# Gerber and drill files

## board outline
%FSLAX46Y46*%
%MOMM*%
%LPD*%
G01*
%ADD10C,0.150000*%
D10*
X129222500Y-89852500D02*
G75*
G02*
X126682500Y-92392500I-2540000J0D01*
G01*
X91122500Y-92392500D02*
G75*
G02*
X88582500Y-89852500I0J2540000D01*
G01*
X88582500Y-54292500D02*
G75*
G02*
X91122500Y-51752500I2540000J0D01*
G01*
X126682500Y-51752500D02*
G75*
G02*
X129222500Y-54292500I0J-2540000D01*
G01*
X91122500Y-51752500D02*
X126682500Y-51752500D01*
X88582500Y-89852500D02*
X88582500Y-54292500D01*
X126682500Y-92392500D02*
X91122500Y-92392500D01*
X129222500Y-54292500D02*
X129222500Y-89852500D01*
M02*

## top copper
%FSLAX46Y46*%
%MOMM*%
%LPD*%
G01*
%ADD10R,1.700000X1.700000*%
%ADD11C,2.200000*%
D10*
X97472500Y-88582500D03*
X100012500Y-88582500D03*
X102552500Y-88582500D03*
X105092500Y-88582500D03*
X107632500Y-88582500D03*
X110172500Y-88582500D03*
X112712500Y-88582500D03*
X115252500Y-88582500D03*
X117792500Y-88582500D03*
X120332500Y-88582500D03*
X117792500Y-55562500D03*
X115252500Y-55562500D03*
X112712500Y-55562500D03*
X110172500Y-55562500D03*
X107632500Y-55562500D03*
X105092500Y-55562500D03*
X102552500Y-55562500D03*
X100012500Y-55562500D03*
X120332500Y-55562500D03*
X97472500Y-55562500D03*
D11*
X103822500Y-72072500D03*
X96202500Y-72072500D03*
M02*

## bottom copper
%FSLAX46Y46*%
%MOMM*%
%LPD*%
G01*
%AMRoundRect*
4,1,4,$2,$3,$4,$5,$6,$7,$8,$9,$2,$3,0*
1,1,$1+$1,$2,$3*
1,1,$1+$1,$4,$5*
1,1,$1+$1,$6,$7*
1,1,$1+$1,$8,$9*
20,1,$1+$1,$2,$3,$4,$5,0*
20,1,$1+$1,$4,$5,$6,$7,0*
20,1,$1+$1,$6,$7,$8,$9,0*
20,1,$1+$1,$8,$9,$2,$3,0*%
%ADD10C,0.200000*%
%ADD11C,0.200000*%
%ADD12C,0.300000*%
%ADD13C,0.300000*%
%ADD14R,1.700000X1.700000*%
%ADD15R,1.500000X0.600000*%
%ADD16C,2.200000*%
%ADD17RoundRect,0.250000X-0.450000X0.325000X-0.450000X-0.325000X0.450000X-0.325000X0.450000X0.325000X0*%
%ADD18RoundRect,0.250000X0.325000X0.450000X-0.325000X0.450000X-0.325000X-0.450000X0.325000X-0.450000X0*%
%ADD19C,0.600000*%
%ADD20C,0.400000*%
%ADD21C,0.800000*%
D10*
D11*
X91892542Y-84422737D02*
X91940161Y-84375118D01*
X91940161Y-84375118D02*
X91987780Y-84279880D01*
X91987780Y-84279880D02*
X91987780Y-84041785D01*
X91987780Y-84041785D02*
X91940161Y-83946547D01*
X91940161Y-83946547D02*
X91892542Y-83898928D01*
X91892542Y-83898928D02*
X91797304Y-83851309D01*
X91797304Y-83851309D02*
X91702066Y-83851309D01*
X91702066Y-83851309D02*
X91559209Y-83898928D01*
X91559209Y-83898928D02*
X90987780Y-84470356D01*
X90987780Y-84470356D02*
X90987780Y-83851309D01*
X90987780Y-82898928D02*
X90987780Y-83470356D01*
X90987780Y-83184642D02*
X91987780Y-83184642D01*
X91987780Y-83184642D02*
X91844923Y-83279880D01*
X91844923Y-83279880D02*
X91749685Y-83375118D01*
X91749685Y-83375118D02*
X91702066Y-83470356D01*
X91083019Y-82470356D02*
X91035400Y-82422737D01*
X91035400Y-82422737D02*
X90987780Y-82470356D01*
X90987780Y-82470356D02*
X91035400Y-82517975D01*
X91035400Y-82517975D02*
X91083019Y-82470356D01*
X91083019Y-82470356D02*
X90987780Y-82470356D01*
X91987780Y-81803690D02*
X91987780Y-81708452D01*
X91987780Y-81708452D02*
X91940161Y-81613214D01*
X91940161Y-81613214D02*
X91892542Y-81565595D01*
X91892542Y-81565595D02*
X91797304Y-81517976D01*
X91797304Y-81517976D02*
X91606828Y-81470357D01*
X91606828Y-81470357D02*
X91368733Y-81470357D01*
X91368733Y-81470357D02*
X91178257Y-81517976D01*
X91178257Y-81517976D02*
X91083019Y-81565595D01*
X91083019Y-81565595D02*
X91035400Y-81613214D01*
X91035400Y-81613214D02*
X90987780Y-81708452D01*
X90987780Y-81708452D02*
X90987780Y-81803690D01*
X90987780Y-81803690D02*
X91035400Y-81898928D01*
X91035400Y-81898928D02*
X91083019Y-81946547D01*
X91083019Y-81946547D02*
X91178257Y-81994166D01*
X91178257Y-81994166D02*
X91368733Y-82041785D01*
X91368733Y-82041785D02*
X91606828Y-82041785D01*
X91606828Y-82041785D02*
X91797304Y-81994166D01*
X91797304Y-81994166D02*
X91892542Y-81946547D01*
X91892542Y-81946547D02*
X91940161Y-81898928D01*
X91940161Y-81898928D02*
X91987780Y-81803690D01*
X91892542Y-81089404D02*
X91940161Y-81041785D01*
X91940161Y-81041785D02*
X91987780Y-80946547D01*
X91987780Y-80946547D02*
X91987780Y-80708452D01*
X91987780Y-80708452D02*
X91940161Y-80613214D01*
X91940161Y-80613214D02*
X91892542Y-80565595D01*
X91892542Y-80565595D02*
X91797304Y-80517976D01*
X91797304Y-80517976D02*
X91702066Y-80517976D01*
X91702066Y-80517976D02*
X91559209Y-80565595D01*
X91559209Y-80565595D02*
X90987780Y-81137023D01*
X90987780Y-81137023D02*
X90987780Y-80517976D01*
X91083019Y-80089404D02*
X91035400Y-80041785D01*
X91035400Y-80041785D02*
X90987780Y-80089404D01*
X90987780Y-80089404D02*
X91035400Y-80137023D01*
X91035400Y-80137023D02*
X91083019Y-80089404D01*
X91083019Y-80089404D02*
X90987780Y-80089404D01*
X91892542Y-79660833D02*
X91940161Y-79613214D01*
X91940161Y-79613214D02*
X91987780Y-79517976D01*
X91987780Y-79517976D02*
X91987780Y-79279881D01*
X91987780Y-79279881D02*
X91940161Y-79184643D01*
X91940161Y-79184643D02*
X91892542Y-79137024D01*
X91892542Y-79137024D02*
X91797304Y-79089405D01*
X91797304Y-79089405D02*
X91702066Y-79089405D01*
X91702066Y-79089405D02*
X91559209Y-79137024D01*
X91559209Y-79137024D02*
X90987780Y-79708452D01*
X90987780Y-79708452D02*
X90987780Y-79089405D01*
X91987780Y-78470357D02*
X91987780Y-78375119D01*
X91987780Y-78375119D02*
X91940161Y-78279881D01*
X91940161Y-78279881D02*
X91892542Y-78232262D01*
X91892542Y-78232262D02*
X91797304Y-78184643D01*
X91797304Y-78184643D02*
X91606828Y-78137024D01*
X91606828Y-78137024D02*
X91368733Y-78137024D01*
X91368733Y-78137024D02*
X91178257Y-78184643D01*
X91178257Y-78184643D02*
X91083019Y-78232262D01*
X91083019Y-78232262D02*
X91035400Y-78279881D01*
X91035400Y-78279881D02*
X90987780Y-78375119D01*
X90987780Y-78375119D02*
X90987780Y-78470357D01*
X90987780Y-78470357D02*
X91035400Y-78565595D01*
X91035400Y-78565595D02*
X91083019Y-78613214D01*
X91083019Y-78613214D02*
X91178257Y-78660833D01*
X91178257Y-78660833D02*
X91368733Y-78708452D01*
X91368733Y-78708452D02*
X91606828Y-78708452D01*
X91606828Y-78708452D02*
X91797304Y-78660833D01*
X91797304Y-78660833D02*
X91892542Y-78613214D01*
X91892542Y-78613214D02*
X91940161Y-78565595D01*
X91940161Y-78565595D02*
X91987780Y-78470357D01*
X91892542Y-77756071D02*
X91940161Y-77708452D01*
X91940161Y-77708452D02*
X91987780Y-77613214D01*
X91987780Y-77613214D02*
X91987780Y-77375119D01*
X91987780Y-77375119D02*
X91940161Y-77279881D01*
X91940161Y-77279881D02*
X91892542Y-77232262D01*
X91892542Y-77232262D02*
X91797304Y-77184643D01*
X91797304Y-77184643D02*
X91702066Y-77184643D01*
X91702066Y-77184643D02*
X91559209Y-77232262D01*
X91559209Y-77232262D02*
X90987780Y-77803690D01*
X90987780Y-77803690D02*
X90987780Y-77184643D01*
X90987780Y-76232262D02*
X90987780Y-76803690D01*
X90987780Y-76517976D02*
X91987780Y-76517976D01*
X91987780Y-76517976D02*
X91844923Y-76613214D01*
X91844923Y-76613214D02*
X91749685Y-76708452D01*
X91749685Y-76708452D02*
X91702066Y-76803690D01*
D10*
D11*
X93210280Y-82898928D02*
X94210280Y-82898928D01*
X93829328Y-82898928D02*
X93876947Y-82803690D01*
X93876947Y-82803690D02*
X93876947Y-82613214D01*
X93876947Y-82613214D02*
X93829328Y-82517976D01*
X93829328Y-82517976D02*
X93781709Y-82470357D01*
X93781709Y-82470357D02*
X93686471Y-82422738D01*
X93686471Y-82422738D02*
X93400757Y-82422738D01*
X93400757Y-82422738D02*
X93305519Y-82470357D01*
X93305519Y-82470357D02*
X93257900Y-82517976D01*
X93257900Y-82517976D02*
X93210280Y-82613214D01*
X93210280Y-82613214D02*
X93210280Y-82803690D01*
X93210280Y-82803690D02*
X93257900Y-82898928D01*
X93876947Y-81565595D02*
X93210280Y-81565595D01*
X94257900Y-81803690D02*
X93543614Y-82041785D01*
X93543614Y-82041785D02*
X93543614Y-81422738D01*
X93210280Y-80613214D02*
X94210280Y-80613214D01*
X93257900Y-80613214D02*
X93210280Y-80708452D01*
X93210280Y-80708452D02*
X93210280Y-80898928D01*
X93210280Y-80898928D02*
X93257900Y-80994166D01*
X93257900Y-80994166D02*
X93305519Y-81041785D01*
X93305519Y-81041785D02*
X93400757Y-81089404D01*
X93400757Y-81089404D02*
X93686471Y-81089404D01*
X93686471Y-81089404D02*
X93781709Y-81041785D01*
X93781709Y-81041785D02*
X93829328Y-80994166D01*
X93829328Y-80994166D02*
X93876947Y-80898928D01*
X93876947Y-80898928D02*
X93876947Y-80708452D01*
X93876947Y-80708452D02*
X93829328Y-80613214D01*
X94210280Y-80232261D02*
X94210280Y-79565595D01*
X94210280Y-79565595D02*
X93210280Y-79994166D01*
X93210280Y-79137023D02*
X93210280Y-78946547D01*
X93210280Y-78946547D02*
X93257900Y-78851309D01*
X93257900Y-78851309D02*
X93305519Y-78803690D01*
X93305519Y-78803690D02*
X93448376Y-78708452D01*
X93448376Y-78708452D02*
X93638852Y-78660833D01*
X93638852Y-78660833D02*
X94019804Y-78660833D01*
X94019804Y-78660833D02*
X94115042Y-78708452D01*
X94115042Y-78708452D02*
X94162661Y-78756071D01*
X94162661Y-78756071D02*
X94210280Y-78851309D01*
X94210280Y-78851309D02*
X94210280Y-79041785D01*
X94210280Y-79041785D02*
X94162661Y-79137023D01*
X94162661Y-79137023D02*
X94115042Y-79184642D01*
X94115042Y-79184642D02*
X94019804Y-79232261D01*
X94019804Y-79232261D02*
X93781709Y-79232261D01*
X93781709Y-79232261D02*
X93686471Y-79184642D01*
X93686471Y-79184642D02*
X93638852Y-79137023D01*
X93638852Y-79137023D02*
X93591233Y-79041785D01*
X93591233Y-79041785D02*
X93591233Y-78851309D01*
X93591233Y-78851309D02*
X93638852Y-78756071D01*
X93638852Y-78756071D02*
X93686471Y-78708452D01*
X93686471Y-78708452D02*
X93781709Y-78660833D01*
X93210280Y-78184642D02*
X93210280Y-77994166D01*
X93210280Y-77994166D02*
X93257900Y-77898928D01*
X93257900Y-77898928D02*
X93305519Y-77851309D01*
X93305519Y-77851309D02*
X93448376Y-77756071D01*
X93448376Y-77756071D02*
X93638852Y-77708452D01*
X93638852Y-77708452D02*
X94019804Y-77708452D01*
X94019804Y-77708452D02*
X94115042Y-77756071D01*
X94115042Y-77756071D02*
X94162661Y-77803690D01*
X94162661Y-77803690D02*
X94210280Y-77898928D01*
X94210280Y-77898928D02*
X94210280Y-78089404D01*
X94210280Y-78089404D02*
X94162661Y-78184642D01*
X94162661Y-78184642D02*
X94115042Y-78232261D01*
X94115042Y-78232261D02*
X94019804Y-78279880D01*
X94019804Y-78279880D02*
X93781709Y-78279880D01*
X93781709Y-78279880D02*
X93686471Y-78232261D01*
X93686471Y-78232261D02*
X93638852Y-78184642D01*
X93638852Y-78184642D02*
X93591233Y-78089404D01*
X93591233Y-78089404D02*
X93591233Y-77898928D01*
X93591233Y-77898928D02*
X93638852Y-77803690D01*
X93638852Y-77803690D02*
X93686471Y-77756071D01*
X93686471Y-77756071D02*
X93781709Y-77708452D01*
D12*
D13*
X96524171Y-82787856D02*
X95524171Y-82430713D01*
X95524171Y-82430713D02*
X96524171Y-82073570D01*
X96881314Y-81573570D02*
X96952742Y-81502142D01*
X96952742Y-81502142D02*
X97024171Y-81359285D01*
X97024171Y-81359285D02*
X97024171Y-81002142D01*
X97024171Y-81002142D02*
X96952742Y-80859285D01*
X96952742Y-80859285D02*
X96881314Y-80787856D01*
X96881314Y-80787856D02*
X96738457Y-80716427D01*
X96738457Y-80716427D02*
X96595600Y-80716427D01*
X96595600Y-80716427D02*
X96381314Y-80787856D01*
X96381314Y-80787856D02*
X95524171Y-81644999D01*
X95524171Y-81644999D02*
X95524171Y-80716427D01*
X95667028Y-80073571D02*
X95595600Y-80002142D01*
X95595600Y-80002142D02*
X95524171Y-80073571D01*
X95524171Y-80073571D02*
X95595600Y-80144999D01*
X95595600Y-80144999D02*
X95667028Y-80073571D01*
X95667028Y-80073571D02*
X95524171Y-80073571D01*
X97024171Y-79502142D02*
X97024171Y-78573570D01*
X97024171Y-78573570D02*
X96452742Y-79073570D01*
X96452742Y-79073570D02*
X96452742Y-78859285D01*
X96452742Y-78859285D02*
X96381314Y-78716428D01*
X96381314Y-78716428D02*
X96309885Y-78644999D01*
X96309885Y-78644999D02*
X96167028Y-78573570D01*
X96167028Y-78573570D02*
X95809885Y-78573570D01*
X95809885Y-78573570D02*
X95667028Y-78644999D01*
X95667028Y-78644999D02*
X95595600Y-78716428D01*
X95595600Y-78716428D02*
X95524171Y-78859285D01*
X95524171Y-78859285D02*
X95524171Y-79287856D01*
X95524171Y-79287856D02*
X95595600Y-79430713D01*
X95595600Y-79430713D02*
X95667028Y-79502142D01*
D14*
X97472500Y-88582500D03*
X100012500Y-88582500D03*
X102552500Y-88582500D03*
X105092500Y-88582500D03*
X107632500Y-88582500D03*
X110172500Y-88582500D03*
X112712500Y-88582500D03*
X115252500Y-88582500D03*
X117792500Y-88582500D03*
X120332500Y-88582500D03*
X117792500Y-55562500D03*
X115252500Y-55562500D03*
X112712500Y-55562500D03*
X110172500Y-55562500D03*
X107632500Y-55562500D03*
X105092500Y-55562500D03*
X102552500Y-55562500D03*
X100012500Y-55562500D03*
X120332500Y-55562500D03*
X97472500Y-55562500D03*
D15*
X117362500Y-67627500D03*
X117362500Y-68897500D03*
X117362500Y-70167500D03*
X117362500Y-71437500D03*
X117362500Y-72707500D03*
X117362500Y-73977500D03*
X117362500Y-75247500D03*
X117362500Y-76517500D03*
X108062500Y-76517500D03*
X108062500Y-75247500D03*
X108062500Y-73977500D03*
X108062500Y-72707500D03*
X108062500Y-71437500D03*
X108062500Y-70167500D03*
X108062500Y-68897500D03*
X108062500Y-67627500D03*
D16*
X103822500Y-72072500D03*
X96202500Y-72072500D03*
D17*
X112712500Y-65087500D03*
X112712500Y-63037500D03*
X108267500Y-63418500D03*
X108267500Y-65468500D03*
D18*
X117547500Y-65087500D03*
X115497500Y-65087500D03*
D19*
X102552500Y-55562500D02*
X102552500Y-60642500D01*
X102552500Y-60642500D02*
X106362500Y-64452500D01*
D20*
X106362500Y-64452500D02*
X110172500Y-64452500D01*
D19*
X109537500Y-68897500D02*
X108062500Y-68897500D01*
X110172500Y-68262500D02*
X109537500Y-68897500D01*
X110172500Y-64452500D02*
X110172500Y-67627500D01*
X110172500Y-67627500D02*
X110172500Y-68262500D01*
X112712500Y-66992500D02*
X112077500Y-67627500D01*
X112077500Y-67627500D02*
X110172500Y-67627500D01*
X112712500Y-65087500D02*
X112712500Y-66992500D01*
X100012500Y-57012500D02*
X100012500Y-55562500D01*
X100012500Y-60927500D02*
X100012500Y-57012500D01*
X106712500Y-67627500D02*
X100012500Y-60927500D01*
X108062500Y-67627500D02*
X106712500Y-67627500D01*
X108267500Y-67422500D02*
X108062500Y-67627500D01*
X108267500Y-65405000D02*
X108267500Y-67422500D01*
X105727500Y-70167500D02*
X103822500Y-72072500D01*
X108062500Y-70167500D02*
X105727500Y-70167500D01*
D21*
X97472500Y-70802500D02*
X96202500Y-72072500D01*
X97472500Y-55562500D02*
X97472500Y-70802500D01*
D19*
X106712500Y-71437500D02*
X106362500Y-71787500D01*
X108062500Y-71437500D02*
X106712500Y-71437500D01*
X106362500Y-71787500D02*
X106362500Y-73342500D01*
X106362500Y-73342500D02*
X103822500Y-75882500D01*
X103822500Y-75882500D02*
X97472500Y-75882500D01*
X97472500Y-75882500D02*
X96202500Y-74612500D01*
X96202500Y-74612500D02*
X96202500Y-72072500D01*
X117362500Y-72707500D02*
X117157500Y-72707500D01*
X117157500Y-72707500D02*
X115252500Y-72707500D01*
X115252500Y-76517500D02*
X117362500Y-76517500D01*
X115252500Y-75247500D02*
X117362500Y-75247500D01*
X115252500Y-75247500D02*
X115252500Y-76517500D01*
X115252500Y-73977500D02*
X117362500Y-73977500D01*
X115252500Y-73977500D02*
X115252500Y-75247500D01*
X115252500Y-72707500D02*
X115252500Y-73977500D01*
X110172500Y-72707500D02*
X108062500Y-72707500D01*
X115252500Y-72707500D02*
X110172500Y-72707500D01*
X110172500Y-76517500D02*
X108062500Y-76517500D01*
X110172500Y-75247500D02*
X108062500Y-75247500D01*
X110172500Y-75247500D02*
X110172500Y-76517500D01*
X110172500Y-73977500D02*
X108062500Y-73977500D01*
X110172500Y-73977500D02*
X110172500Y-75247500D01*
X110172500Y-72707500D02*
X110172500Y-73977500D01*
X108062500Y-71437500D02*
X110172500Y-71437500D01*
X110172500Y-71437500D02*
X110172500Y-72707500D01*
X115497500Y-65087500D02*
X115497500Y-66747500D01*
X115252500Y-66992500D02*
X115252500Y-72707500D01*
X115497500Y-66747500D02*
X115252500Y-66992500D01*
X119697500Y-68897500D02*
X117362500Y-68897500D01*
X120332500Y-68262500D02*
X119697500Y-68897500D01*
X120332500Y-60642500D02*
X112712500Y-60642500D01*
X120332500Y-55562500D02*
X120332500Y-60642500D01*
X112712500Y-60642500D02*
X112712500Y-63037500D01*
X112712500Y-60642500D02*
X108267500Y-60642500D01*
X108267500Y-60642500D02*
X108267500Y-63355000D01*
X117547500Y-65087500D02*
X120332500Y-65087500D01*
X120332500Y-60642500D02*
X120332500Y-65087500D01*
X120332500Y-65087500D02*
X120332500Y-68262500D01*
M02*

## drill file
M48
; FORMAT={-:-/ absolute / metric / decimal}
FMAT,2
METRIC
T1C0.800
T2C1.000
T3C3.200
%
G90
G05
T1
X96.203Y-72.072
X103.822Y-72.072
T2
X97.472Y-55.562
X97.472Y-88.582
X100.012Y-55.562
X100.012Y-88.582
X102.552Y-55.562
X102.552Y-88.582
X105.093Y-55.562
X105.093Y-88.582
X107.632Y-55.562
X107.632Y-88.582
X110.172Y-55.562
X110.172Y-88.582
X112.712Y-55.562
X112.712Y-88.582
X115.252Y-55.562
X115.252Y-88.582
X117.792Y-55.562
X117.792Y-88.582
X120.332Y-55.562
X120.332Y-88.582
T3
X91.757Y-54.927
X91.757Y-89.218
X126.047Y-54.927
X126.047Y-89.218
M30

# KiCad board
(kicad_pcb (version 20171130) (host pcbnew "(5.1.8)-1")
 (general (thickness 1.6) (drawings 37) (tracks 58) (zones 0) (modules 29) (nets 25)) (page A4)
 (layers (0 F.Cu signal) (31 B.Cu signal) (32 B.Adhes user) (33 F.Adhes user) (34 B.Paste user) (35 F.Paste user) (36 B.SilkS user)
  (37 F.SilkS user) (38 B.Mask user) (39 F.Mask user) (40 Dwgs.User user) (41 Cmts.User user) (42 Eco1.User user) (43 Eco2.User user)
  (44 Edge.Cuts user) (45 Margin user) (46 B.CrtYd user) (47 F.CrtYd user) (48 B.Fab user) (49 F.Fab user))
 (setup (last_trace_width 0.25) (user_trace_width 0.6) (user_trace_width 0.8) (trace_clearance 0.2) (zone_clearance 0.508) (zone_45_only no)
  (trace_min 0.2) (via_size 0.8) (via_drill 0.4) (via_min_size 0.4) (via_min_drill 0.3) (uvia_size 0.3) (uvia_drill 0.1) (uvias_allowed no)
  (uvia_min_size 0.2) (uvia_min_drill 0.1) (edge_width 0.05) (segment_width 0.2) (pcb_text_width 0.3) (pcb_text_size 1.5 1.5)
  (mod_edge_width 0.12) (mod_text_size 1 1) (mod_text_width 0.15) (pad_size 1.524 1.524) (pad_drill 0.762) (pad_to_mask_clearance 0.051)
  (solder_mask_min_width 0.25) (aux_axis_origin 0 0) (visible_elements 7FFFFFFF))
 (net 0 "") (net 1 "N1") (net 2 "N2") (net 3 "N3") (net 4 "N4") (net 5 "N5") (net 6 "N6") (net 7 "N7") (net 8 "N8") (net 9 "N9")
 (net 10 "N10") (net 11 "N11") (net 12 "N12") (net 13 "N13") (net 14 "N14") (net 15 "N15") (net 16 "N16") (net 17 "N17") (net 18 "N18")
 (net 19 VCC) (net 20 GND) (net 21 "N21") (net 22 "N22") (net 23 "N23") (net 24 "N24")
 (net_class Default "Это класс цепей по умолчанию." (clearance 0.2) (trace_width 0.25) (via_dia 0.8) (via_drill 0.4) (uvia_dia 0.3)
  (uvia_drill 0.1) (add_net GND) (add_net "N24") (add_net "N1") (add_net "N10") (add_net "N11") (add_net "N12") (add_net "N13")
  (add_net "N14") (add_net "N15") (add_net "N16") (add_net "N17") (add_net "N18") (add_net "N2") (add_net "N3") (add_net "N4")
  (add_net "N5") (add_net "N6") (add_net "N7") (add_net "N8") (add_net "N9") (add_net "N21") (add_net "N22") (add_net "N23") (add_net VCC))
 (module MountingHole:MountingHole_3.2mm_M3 (layer F.Cu) (at 126.0475 54.9275 270)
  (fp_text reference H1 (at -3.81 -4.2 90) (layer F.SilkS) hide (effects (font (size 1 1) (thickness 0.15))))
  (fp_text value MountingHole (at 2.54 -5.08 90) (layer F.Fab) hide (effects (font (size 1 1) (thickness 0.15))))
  (pad 1 np_thru_hole circle (at 0 0 270) (size 3.2 3.2) (drill 3.2) (layers *.Cu *.Mask)))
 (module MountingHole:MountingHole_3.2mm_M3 (layer F.Cu) (at 91.7575 54.9275 270)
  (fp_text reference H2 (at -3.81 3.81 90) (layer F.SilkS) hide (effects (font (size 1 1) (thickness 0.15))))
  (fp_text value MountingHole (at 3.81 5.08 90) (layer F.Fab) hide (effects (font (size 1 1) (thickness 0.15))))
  (pad 1 np_thru_hole circle (at 0 0 270) (size 3.2 3.2) (drill 3.2) (layers *.Cu *.Mask)))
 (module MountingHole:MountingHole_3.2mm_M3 (layer F.Cu) (at 126.0475 89.2175 270)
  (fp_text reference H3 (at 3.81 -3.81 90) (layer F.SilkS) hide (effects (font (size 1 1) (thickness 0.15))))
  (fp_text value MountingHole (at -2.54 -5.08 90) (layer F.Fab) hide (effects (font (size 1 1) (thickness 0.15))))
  (pad 1 np_thru_hole circle (at 0 0 270) (size 3.2 3.2) (drill 3.2) (layers *.Cu *.Mask)))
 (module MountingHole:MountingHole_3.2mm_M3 (layer F.Cu) (at 91.7575 89.2175 270)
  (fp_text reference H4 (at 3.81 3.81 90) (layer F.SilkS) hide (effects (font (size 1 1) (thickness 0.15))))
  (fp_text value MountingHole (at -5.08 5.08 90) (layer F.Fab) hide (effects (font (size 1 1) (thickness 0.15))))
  (pad 1 np_thru_hole circle (at 0 0 270) (size 3.2 3.2) (drill 3.2) (layers *.Cu *.Mask)))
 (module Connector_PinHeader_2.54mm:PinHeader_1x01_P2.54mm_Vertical (layer F.Cu) (at 97.4725 88.5825 270)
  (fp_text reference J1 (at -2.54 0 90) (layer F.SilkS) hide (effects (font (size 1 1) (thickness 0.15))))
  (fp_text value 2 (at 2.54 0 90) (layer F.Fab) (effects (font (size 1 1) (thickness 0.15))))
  (pad 1 thru_hole rect (at 0 0 270) (size 1.7 1.7) (drill 1) (layers *.Cu *.Mask) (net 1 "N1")))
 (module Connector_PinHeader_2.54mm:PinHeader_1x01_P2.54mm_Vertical (layer F.Cu) (at 100.0125 88.5825 270)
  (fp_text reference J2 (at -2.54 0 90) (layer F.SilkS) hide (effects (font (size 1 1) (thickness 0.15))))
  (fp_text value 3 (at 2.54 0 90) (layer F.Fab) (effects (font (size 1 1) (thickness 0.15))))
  (pad 1 thru_hole rect (at 0 0 270) (size 1.7 1.7) (drill 1) (layers *.Cu *.Mask) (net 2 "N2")))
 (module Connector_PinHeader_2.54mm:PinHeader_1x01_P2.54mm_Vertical (layer F.Cu) (at 102.5525 88.5825 270)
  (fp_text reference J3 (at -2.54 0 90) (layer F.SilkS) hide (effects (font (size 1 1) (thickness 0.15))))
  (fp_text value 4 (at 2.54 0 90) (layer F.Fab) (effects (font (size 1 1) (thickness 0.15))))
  (pad 1 thru_hole rect (at 0 0 270) (size 1.7 1.7) (drill 1) (layers *.Cu *.Mask) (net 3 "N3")))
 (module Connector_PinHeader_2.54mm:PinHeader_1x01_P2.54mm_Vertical (layer F.Cu) (at 105.0925 88.5825 270)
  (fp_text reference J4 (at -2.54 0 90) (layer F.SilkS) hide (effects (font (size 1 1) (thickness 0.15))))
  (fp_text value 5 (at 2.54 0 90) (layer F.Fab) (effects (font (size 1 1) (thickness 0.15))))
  (pad 1 thru_hole rect (at 0 0 270) (size 1.7 1.7) (drill 1) (layers *.Cu *.Mask) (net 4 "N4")))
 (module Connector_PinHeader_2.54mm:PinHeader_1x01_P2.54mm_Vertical (layer F.Cu) (at 107.6325 88.5825 270)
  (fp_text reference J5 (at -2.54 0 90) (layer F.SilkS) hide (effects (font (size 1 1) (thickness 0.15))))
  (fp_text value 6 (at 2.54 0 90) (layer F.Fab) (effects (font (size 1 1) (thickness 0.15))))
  (pad 1 thru_hole rect (at 0 0 270) (size 1.7 1.7) (drill 1) (layers *.Cu *.Mask) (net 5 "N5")))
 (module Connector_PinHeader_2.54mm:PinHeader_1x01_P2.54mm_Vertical (layer F.Cu) (at 110.1725 88.5825 270)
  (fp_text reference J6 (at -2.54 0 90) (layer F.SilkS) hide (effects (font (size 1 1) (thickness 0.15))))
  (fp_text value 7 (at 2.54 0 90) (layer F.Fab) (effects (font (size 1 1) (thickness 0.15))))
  (pad 1 thru_hole rect (at 0 0 270) (size 1.7 1.7) (drill 1) (layers *.Cu *.Mask) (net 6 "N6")))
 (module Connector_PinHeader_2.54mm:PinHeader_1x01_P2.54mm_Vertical (layer F.Cu) (at 112.7125 88.5825 270)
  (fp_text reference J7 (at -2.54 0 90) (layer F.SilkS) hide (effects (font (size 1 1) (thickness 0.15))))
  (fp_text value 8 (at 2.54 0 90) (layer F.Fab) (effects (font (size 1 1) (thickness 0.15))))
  (pad 1 thru_hole rect (at 0 0 270) (size 1.7 1.7) (drill 1) (layers *.Cu *.Mask) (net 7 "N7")))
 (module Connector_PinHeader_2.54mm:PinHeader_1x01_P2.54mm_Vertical (layer F.Cu) (at 115.2525 88.5825 270)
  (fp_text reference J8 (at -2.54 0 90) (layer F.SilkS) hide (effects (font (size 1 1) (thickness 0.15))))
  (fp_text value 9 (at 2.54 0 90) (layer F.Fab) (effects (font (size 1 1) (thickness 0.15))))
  (pad 1 thru_hole rect (at 0 0 270) (size 1.7 1.7) (drill 1) (layers *.Cu *.Mask) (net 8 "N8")))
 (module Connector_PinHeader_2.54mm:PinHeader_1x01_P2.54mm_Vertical (layer F.Cu) (at 117.7925 88.5825 270)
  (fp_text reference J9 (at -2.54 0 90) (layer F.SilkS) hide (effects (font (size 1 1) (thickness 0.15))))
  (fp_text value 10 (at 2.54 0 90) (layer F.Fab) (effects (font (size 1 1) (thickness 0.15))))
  (pad 1 thru_hole rect (at 0 0 270) (size 1.7 1.7) (drill 1) (layers *.Cu *.Mask) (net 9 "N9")))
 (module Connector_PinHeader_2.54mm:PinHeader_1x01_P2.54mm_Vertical (layer F.Cu) (at 120.3325 88.5825 270)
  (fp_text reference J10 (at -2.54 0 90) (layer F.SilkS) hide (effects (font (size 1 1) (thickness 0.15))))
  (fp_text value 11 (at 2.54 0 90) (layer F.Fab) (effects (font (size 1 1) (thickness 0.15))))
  (pad 1 thru_hole rect (at 0 0 270) (size 1.7 1.7) (drill 1) (layers *.Cu *.Mask) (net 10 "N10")))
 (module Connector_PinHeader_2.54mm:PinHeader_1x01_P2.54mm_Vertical (layer F.Cu) (at 117.7925 55.5625 270)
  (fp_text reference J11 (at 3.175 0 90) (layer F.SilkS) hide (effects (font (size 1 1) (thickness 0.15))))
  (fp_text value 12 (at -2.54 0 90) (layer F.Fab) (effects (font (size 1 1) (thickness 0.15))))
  (pad 1 thru_hole rect (at 0 0 270) (size 1.7 1.7) (drill 1) (layers *.Cu *.Mask) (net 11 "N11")))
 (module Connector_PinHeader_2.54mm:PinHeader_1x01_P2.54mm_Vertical (layer F.Cu) (at 115.2525 55.5625 270)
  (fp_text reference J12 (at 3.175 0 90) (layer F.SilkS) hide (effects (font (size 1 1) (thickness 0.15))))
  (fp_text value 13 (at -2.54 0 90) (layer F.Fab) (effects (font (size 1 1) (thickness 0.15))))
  (pad 1 thru_hole rect (at 0 0 270) (size 1.7 1.7) (drill 1) (layers *.Cu *.Mask) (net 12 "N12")))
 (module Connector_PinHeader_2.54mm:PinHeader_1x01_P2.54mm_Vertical (layer F.Cu) (at 112.7125 55.5625 270)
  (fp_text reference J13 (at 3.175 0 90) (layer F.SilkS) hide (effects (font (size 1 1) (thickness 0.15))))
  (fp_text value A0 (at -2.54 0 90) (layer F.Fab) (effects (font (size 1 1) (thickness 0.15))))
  (pad 1 thru_hole rect (at 0 0 270) (size 1.7 1.7) (drill 1) (layers *.Cu *.Mask) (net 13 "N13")))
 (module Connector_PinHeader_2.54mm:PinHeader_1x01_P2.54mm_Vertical (layer F.Cu) (at 110.1725 55.5625 270)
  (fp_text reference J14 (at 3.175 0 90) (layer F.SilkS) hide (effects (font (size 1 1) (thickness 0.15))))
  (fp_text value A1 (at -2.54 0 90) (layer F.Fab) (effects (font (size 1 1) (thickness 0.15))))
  (pad 1 thru_hole rect (at 0 0 270) (size 1.7 1.7) (drill 1) (layers *.Cu *.Mask) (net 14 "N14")))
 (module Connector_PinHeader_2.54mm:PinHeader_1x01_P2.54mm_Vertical (layer F.Cu) (at 107.6325 55.5625 270)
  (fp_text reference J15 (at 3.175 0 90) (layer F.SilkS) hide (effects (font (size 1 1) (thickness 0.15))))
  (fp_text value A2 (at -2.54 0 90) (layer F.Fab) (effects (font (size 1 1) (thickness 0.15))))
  (pad 1 thru_hole rect (at 0 0 270) (size 1.7 1.7) (drill 1) (layers *.Cu *.Mask) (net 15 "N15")))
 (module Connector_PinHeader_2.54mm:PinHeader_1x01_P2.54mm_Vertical (layer F.Cu) (at 105.0925 55.5625 270)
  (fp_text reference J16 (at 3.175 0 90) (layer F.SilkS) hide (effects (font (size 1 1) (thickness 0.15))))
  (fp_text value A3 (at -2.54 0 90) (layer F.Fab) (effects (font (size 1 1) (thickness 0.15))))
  (pad 1 thru_hole rect (at 0 0 270) (size 1.7 1.7) (drill 1) (layers *.Cu *.Mask) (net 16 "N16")))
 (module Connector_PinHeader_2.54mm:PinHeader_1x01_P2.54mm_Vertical (layer F.Cu) (at 102.5525 55.5625 270)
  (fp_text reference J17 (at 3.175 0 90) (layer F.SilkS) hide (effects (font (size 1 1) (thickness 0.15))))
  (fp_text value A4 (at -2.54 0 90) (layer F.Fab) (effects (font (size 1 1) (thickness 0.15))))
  (pad 1 thru_hole rect (at 0 0 270) (size 1.7 1.7) (drill 1) (layers *.Cu *.Mask) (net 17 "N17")))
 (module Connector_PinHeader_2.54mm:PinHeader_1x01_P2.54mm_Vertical (layer F.Cu) (at 100.0125 55.5625 270)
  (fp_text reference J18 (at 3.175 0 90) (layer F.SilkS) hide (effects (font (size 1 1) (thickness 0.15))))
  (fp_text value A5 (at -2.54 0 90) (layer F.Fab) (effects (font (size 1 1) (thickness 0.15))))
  (pad 1 thru_hole rect (at 0 0 270) (size 1.7 1.7) (drill 1) (layers *.Cu *.Mask) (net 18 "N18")))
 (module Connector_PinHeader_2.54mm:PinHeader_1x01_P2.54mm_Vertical (layer F.Cu) (at 120.3325 55.5625 270)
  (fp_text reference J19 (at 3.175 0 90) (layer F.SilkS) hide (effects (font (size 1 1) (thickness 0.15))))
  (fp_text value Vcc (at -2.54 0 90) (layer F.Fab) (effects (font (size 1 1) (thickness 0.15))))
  (pad 1 thru_hole rect (at 0 0 270) (size 1.7 1.7) (drill 1) (layers *.Cu *.Mask) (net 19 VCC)))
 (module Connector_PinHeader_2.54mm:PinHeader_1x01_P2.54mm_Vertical (layer F.Cu) (at 97.4725 55.5625 270)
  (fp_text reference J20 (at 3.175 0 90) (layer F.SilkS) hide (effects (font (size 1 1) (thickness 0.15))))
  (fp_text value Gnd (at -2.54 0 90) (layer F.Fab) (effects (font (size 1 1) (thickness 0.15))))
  (pad 1 thru_hole rect (at 0 0 270) (size 1.7 1.7) (drill 1) (layers *.Cu *.Mask) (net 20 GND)))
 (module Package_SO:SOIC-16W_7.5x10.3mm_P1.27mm (layer B.Cu) (at 112.7125 72.0725 180)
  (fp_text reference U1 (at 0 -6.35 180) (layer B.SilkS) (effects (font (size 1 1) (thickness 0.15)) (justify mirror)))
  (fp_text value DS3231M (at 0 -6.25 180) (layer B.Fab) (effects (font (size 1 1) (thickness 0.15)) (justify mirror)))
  (pad 1 smd rect (at -4.65 4.445 180) (size 1.5 0.6) (layers B.Cu B.Paste B.Mask) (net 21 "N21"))
  (pad 2 smd rect (at -4.65 3.175 180) (size 1.5 0.6) (layers B.Cu B.Paste B.Mask) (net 19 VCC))
  (pad 3 smd rect (at -4.65 1.905 180) (size 1.5 0.6) (layers B.Cu B.Paste B.Mask) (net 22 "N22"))
  (pad 4 smd rect (at -4.65 0.635 180) (size 1.5 0.6) (layers B.Cu B.Paste B.Mask) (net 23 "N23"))
  (pad 5 smd rect (at -4.65 -0.635 180) (size 1.5 0.6) (layers B.Cu B.Paste B.Mask) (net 20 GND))
  (pad 6 smd rect (at -4.65 -1.905 180) (size 1.5 0.6) (layers B.Cu B.Paste B.Mask) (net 20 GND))
  (pad 7 smd rect (at -4.65 -3.175 180) (size 1.5 0.6) (layers B.Cu B.Paste B.Mask) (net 20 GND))
  (pad 8 smd rect (at -4.65 -4.445 180) (size 1.5 0.6) (layers B.Cu B.Paste B.Mask) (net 20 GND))
  (pad 9 smd rect (at 4.65 -4.445 180) (size 1.5 0.6) (layers B.Cu B.Paste B.Mask) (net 20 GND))
  (pad 10 smd rect (at 4.65 -3.175 180) (size 1.5 0.6) (layers B.Cu B.Paste B.Mask) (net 20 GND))
  (pad 11 smd rect (at 4.65 -1.905 180) (size 1.5 0.6) (layers B.Cu B.Paste B.Mask) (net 20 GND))
  (pad 12 smd rect (at 4.65 -0.635 180) (size 1.5 0.6) (layers B.Cu B.Paste B.Mask) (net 20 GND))
  (pad 13 smd rect (at 4.65 0.635 180) (size 1.5 0.6) (layers B.Cu B.Paste B.Mask) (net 20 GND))
  (pad 14 smd rect (at 4.65 1.905 180) (size 1.5 0.6) (layers B.Cu B.Paste B.Mask) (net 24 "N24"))
  (pad 15 smd rect (at 4.65 3.175 180) (size 1.5 0.6) (layers B.Cu B.Paste B.Mask) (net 17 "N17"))
  (pad 16 smd rect (at 4.65 4.445 180) (size 1.5 0.6) (layers B.Cu B.Paste B.Mask) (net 18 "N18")))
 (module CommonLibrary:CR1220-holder (layer F.Cu) (at 96.2025 72.0725 180)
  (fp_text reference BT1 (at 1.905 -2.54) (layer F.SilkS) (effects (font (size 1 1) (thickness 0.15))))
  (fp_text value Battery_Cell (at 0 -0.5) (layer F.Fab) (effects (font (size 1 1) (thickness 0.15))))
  (pad 1 thru_hole circle (at -7.62 0 180) (size 2.2 2.2) (drill 0.8) (layers *.Cu *.Mask) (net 24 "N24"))
  (pad 2 thru_hole circle (at 0 0 180) (size 2.2 2.2) (drill 0.8) (layers *.Cu *.Mask) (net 20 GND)))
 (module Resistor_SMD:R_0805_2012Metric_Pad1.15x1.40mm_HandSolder (layer B.Cu) (at 112.7125 64.0625 270)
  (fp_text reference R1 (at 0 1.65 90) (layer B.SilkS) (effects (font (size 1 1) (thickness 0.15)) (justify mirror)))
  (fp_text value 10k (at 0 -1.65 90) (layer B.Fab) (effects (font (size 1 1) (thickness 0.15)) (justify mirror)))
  (pad 2 smd roundrect (at 1.025 0 270) (size 1.15 1.4) (layers B.Cu B.Paste B.Mask) (roundrect_rratio 0.217391) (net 17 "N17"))
  (pad 1 smd roundrect (at -1.025 0 270) (size 1.15 1.4) (layers B.Cu B.Paste B.Mask) (roundrect_rratio 0.217391) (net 19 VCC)))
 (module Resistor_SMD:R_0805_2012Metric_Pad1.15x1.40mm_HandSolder (layer B.Cu) (at 108.2675 64.4435 270)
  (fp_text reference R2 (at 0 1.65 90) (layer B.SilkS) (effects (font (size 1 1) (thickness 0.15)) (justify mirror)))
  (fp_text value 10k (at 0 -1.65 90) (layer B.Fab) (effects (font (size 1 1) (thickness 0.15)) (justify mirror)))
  (pad 1 smd roundrect (at -1.025 0 270) (size 1.15 1.4) (layers B.Cu B.Paste B.Mask) (roundrect_rratio 0.217391) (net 19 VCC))
  (pad 2 smd roundrect (at 1.025 0 270) (size 1.15 1.4) (layers B.Cu B.Paste B.Mask) (roundrect_rratio 0.217391) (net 18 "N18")))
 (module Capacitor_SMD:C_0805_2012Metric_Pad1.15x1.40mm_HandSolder (layer B.Cu) (at 116.5225 65.0875 180)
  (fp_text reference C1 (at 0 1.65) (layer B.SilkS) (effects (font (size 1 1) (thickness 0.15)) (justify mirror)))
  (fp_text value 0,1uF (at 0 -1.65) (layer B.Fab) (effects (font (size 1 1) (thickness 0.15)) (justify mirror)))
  (pad 1 smd roundrect (at -1.025 0 180) (size 1.15 1.4) (layers B.Cu B.Paste B.Mask) (roundrect_rratio 0.217391) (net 19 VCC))
  (pad 2 smd roundrect (at 1.025 0 180) (size 1.15 1.4) (layers B.Cu B.Paste B.Mask) (roundrect_rratio 0.217391) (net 20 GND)))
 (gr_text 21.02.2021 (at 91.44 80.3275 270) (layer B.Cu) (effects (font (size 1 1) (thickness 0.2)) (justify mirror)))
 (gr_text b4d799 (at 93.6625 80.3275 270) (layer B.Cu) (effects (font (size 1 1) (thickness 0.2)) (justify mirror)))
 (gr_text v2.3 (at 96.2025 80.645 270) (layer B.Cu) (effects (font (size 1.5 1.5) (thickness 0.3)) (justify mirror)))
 (gr_arc (start 126.6825 89.8525) (end 126.6825 92.3925) (angle -90) (layer Edge.Cuts) (width 0.15))
 (gr_arc (start 91.1225 89.8525) (end 88.5825 89.8525) (angle -90) (layer Edge.Cuts) (width 0.15))
 (gr_arc (start 91.1225 54.2925) (end 91.1225 51.7525) (angle -90) (layer Edge.Cuts) (width 0.15))
 (gr_arc (start 126.6825 54.2925) (end 129.2225 54.2925) (angle -90) (layer Edge.Cuts) (width 0.15))
 (gr_line (start 91.1225 51.7525) (end 126.6825 51.7525) (layer Edge.Cuts) (width 0.15))
 (gr_line (start 88.5825 89.8525) (end 88.5825 54.2925) (layer Edge.Cuts) (width 0.15))
 (gr_line (start 126.6825 92.3925) (end 91.1225 92.3925) (layer Edge.Cuts) (width 0.15))
 (gr_line (start 129.2225 54.2925) (end 129.2225 89.8525) (layer Edge.Cuts) (width 0.15))
 (segment (start 102.5525 55.5625) (end 102.5525 60.6425) (width 0.6) (layer B.Cu) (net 17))
 (segment (start 102.5525 60.6425) (end 106.3625 64.4525) (width 0.6) (layer B.Cu) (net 17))
 (segment (start 106.3625 64.4525) (end 110.1725 64.4525) (width 0.4) (layer B.Cu) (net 17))
 (segment (start 109.5375 68.8975) (end 108.0625 68.8975) (width 0.6) (layer B.Cu) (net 17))
 (segment (start 110.1725 68.2625) (end 109.5375 68.8975) (width 0.6) (layer B.Cu) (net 17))
 (segment (start 110.1725 64.4525) (end 110.1725 67.6275) (width 0.6) (layer B.Cu) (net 17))
 (segment (start 110.1725 67.6275) (end 110.1725 68.2625) (width 0.6) (layer B.Cu) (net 17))
 (segment (start 112.7125 66.9925) (end 112.0775 67.6275) (width 0.6) (layer B.Cu) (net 17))
 (segment (start 112.0775 67.6275) (end 110.1725 67.6275) (width 0.6) (layer B.Cu) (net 17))
 (segment (start 112.7125 65.0875) (end 112.7125 66.9925) (width 0.6) (layer B.Cu) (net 17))
 (segment (start 100.0125 57.0125) (end 100.0125 55.5625) (width 0.6) (layer B.Cu) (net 18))
 (segment (start 100.0125 60.9275) (end 100.0125 57.0125) (width 0.6) (layer B.Cu) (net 18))
 (segment (start 106.7125 67.6275) (end 100.0125 60.9275) (width 0.6) (layer B.Cu) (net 18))
 (segment (start 108.0625 67.6275) (end 106.7125 67.6275) (width 0.6) (layer B.Cu) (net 18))
 (segment (start 108.2675 67.4225) (end 108.0625 67.6275) (width 0.6) (layer B.Cu) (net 18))
 (segment (start 108.2675 65.405) (end 108.2675 67.4225) (width 0.6) (layer B.Cu) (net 18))
 (segment (start 105.7275 70.1675) (end 103.8225 72.0725) (width 0.6) (layer B.Cu) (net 24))
 (segment (start 108.0625 70.1675) (end 105.7275 70.1675) (width 0.6) (layer B.Cu) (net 24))
 (segment (start 97.4725 70.8025) (end 96.2025 72.0725) (width 0.8) (layer B.Cu) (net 20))
 (segment (start 97.4725 55.5625) (end 97.4725 70.8025) (width 0.8) (layer B.Cu) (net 20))
 (segment (start 106.7125 71.4375) (end 106.3625 71.7875) (width 0.6) (layer B.Cu) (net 20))
 (segment (start 108.0625 71.4375) (end 106.7125 71.4375) (width 0.6) (layer B.Cu) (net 20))
 (segment (start 106.3625 71.7875) (end 106.3625 73.3425) (width 0.6) (layer B.Cu) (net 20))
 (segment (start 106.3625 73.3425) (end 103.8225 75.8825) (width 0.6) (layer B.Cu) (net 20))
 (segment (start 103.8225 75.8825) (end 97.4725 75.8825) (width 0.6) (layer B.Cu) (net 20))
 (segment (start 97.4725 75.8825) (end 96.2025 74.6125) (width 0.6) (layer B.Cu) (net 20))
 (segment (start 96.2025 74.6125) (end 96.2025 72.0725) (width 0.6) (layer B.Cu) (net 20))
 (segment (start 117.3625 72.7075) (end 117.1575 72.7075) (width 0.6) (layer B.Cu) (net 20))
 (segment (start 117.1575 72.7075) (end 115.2525 72.7075) (width 0.6) (layer B.Cu) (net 20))
 (segment (start 115.2525 76.5175) (end 117.3625 76.5175) (width 0.6) (layer B.Cu) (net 20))
 (segment (start 115.2525 75.2475) (end 117.3625 75.2475) (width 0.6) (layer B.Cu) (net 20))
 (segment (start 115.2525 75.2475) (end 115.2525 76.5175) (width 0.6) (layer B.Cu) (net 20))
 (segment (start 115.2525 73.9775) (end 117.3625 73.9775) (width 0.6) (layer B.Cu) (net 20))
 (segment (start 115.2525 73.9775) (end 115.2525 75.2475) (width 0.6) (layer B.Cu) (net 20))
 (segment (start 115.2525 72.7075) (end 115.2525 73.9775) (width 0.6) (layer B.Cu) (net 20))
 (segment (start 110.1725 72.7075) (end 108.0625 72.7075) (width 0.6) (layer B.Cu) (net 20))
 (segment (start 115.2525 72.7075) (end 110.1725 72.7075) (width 0.6) (layer B.Cu) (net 20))
 (segment (start 110.1725 76.5175) (end 108.0625 76.5175) (width 0.6) (layer B.Cu) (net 20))
 (segment (start 110.1725 75.2475) (end 108.0625 75.2475) (width 0.6) (layer B.Cu) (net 20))
 (segment (start 110.1725 75.2475) (end 110.1725 76.5175) (width 0.6) (layer B.Cu) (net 20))
 (segment (start 110.1725 73.9775) (end 108.0625 73.9775) (width 0.6) (layer B.Cu) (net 20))
 (segment (start 110.1725 73.9775) (end 110.1725 75.2475) (width 0.6) (layer B.Cu) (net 20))
 (segment (start 110.1725 72.7075) (end 110.1725 73.9775) (width 0.6) (layer B.Cu) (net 20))
 (segment (start 108.0625 71.4375) (end 110.1725 71.4375) (width 0.6) (layer B.Cu) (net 20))
 (segment (start 110.1725 71.4375) (end 110.1725 72.7075) (width 0.6) (layer B.Cu) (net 20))
 (segment (start 115.4975 65.0875) (end 115.4975 66.7475) (width 0.6) (layer B.Cu) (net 20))
 (segment (start 115.2525 66.9925) (end 115.2525 72.7075) (width 0.6) (layer B.Cu) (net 20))
 (segment (start 115.4975 66.7475) (end 115.2525 66.9925) (width 0.6) (layer B.Cu) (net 20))
 (segment (start 119.6975 68.8975) (end 117.3625 68.8975) (width 0.6) (layer B.Cu) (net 19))
 (segment (start 120.3325 68.2625) (end 119.6975 68.8975) (width 0.6) (layer B.Cu) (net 19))
 (segment (start 120.3325 60.6425) (end 112.7125 60.6425) (width 0.6) (layer B.Cu) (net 19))
 (segment (start 120.3325 55.5625) (end 120.3325 60.6425) (width 0.6) (layer B.Cu) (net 19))
 (segment (start 112.7125 60.6425) (end 112.7125 63.0375) (width 0.6) (layer B.Cu) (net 19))
 (segment (start 112.7125 60.6425) (end 108.2675 60.6425) (width 0.6) (layer B.Cu) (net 19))
 (segment (start 108.2675 60.6425) (end 108.2675 63.355) (width 0.6) (layer B.Cu) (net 19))
 (segment (start 117.5475 65.0875) (end 120.3325 65.0875) (width 0.6) (layer B.Cu) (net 19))
 (segment (start 120.3325 60.6425) (end 120.3325 65.0875) (width 0.6) (layer B.Cu) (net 19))
 (segment (start 120.3325 65.0875) (end 120.3325 68.2625) (width 0.6) (layer B.Cu) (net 19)))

